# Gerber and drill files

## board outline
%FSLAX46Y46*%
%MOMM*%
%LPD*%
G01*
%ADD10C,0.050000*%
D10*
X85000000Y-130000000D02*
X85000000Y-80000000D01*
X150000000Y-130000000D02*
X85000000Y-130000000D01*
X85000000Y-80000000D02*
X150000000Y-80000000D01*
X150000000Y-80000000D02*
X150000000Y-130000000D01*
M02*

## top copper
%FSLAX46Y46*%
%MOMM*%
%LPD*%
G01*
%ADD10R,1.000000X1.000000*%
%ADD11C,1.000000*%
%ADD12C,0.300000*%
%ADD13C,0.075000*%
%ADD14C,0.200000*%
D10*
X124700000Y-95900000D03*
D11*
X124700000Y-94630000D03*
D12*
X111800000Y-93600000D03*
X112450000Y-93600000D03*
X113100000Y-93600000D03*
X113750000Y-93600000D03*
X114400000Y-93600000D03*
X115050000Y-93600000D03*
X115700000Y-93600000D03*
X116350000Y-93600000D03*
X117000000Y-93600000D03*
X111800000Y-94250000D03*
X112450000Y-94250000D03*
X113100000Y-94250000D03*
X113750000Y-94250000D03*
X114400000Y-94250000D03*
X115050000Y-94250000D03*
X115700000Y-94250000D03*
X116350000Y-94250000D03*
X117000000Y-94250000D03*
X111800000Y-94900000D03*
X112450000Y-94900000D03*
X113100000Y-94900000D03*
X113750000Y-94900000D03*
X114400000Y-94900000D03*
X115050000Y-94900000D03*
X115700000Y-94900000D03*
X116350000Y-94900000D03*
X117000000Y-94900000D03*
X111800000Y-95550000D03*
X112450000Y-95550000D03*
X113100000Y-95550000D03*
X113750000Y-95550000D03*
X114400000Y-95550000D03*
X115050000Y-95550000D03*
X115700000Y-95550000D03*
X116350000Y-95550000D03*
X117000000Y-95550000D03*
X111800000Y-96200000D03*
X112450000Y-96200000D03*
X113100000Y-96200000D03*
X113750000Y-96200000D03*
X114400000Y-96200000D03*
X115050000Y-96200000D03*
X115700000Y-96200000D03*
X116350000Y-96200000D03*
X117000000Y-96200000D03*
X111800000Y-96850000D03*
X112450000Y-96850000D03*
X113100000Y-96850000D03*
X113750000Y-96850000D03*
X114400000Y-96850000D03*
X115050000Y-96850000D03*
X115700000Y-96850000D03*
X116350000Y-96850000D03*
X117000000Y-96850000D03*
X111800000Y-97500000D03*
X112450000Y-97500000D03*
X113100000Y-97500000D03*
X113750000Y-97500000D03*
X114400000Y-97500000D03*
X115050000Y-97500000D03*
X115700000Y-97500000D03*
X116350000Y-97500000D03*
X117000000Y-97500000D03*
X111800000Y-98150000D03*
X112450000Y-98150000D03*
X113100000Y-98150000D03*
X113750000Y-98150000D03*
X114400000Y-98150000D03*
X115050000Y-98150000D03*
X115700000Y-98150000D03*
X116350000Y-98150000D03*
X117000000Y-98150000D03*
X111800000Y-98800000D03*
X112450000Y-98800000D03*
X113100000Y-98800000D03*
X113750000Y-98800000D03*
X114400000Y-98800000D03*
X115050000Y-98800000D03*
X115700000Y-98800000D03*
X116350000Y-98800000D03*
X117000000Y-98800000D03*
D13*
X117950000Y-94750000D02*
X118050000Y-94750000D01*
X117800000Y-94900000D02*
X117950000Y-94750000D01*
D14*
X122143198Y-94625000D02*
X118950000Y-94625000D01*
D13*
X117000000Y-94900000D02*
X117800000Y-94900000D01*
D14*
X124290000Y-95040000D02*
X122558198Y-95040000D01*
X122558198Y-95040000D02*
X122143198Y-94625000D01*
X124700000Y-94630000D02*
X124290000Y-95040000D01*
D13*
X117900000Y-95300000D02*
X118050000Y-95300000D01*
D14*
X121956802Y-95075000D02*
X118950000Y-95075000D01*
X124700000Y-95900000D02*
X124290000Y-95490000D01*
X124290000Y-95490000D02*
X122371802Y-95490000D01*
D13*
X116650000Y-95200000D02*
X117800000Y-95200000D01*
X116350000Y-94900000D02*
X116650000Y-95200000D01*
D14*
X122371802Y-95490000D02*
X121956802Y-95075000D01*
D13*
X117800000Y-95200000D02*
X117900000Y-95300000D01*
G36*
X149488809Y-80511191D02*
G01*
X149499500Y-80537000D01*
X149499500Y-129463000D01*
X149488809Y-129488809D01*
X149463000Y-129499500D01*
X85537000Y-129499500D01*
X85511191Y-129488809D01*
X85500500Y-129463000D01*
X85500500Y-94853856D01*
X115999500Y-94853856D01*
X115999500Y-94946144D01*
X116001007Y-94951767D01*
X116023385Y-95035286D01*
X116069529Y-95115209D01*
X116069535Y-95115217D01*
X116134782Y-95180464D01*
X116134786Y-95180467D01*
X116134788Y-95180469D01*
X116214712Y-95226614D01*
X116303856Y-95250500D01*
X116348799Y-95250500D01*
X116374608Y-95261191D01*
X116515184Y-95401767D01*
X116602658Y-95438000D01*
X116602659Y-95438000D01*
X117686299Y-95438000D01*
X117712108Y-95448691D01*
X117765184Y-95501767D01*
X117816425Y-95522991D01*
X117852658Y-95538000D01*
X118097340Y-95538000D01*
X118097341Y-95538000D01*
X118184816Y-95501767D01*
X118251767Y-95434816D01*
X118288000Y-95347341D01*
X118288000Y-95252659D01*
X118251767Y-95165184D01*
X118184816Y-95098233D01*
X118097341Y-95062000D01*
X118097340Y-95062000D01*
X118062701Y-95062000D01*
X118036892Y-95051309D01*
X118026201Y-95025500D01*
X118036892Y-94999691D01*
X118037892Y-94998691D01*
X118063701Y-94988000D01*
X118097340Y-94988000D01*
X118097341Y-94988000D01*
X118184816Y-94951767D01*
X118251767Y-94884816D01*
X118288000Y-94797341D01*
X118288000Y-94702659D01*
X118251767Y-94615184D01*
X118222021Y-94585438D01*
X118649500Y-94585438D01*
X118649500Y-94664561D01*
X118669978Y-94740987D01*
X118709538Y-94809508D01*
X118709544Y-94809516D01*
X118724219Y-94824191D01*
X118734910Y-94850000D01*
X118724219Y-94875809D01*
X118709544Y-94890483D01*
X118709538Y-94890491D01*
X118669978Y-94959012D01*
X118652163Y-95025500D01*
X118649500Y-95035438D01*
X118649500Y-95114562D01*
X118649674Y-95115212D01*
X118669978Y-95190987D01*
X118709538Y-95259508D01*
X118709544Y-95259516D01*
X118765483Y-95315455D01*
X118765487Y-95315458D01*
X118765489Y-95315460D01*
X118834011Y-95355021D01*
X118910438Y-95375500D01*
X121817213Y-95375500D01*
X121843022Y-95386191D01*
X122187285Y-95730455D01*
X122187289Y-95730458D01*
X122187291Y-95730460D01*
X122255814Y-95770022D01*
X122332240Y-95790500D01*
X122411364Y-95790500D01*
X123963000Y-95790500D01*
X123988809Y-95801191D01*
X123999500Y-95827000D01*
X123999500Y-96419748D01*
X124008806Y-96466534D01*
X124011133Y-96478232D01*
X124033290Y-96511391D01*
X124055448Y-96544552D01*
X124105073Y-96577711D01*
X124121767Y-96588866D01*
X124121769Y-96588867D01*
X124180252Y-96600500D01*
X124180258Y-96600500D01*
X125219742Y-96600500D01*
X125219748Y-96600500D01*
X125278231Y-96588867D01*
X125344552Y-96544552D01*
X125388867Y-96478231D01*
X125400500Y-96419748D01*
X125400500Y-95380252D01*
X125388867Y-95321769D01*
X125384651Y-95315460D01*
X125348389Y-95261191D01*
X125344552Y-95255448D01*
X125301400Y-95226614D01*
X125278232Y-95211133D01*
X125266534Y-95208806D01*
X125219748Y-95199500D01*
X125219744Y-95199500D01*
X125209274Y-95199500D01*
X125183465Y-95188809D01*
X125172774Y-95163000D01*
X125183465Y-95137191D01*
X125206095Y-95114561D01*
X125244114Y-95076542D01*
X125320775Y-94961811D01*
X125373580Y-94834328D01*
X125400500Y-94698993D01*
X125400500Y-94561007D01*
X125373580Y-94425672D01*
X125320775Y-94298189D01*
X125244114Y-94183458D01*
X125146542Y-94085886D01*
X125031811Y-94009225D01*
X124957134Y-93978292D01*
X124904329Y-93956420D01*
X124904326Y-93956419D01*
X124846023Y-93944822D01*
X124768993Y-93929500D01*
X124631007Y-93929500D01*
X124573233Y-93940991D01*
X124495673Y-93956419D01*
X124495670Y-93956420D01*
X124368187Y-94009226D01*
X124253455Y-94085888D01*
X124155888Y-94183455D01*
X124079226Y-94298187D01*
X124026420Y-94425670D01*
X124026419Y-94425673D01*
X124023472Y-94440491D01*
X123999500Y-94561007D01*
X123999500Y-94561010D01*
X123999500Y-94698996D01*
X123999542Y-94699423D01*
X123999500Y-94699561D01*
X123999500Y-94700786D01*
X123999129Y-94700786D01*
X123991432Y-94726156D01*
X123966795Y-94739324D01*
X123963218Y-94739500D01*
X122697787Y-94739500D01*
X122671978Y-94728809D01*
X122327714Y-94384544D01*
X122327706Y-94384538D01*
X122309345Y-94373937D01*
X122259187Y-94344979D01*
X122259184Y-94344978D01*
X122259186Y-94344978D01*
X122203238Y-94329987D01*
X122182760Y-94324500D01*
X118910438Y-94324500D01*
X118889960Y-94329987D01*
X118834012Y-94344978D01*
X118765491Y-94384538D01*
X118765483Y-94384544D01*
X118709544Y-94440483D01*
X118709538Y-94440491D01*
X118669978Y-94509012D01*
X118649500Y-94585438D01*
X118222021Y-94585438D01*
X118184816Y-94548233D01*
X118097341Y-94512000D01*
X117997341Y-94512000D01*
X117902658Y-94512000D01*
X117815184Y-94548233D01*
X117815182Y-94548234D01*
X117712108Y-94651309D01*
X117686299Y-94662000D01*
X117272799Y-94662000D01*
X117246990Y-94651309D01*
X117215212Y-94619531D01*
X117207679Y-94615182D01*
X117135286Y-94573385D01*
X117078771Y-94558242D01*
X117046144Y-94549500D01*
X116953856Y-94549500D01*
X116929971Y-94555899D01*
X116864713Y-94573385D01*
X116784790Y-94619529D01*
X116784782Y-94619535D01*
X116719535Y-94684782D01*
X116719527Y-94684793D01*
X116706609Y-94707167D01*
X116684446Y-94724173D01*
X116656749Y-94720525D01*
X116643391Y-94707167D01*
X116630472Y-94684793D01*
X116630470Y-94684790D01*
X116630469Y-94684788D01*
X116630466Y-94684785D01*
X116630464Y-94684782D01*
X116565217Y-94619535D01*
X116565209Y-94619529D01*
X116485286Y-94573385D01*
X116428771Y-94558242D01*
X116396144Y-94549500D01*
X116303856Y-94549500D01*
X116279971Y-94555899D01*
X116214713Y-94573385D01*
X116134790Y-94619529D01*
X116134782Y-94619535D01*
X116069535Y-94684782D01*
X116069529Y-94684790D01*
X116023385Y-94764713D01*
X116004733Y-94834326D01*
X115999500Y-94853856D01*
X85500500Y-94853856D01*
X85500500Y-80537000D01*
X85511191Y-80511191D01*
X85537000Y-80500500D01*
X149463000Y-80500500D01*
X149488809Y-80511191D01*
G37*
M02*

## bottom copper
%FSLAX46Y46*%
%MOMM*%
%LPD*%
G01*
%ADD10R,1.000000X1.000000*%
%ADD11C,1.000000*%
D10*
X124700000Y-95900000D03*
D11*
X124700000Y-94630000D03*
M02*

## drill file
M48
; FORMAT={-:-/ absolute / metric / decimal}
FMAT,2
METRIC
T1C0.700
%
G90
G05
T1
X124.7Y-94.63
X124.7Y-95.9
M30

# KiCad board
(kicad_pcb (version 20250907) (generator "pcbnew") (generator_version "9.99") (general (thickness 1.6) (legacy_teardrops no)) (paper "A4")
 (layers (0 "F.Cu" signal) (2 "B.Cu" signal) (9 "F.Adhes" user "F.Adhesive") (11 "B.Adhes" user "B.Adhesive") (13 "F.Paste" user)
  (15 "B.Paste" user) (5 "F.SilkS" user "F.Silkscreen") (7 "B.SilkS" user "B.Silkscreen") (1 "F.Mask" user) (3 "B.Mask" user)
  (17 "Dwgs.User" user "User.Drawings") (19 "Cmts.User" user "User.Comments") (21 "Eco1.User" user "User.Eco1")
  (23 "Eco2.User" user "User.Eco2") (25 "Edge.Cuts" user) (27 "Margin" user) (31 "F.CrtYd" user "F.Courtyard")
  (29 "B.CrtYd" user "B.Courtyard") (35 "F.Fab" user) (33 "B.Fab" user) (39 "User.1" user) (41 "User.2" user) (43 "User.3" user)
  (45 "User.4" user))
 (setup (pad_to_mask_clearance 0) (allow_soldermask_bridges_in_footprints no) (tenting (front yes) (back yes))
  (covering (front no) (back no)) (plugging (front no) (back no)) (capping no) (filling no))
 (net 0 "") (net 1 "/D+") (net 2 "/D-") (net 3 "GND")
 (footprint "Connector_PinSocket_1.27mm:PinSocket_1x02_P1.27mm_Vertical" (layer "F.Cu") (at 124.7 95.9 180)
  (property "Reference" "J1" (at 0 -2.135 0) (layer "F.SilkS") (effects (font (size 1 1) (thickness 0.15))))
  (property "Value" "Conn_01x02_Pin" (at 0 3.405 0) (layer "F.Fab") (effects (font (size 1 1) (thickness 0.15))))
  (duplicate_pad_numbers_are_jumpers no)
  (pad "1" thru_hole rect (at 0 0 180) (size 1 1) (drill 0.7) (layers "*.Cu" "*.Mask") (remove_unused_layers no) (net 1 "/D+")
   (tenting (front none) (back none)))
  (pad "2" thru_hole circle (at 0 1.27 180) (size 1 1) (drill 0.7) (layers "*.Cu" "*.Mask") (remove_unused_layers no) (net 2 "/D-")
   (tenting (front none) (back none))))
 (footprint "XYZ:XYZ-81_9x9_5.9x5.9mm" (layer "F.Cu") (at 114.4 96.2)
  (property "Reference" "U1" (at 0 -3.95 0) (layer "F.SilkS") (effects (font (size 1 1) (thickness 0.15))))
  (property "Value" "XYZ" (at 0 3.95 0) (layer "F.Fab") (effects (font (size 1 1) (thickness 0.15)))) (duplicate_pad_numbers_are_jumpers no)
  (pad "A1" smd circle (at -2.6 -2.6) (size 0.3 0.3) (layers "F.Cu" "F.Mask" "F.Paste") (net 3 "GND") (tenting (front none) (back none)))
  (pad "A2" smd circle (at -1.95 -2.6) (size 0.3 0.3) (layers "F.Cu" "F.Mask" "F.Paste") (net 3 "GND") (tenting (front none) (back none)))
  (pad "A3" smd circle (at -1.3 -2.6) (size 0.3 0.3) (layers "F.Cu" "F.Mask" "F.Paste") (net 3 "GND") (tenting (front none) (back none)))
  (pad "A4" smd circle (at -0.65 -2.6) (size 0.3 0.3) (layers "F.Cu" "F.Mask" "F.Paste") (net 3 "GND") (tenting (front none) (back none)))
  (pad "A5" smd circle (at 0 -2.6) (size 0.3 0.3) (layers "F.Cu" "F.Mask" "F.Paste") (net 3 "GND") (tenting (front none) (back none)))
  (pad "A6" smd circle (at 0.65 -2.6) (size 0.3 0.3) (layers "F.Cu" "F.Mask" "F.Paste") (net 3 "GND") (tenting (front none) (back none)))
  (pad "A7" smd circle (at 1.3 -2.6) (size 0.3 0.3) (layers "F.Cu" "F.Mask" "F.Paste") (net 3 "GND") (tenting (front none) (back none)))
  (pad "A8" smd circle (at 1.95 -2.6) (size 0.3 0.3) (layers "F.Cu" "F.Mask" "F.Paste") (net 3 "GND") (tenting (front none) (back none)))
  (pad "A9" smd circle (at 2.6 -2.6) (size 0.3 0.3) (layers "F.Cu" "F.Mask" "F.Paste") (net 3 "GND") (tenting (front none) (back none)))
  (pad "B1" smd circle (at -2.6 -1.95) (size 0.3 0.3) (layers "F.Cu" "F.Mask" "F.Paste") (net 3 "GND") (tenting (front none) (back none)))
  (pad "B2" smd circle (at -1.95 -1.95) (size 0.3 0.3) (layers "F.Cu" "F.Mask" "F.Paste") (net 3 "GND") (tenting (front none) (back none)))
  (pad "B3" smd circle (at -1.3 -1.95) (size 0.3 0.3) (layers "F.Cu" "F.Mask" "F.Paste") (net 3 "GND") (tenting (front none) (back none)))
  (pad "B4" smd circle (at -0.65 -1.95) (size 0.3 0.3) (layers "F.Cu" "F.Mask" "F.Paste") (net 3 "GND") (tenting (front none) (back none)))
  (pad "B5" smd circle (at 0 -1.95) (size 0.3 0.3) (layers "F.Cu" "F.Mask" "F.Paste") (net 3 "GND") (tenting (front none) (back none)))
  (pad "B6" smd circle (at 0.65 -1.95) (size 0.3 0.3) (layers "F.Cu" "F.Mask" "F.Paste") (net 3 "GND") (tenting (front none) (back none)))
  (pad "B7" smd circle (at 1.3 -1.95) (size 0.3 0.3) (layers "F.Cu" "F.Mask" "F.Paste") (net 3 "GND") (tenting (front none) (back none)))
  (pad "B8" smd circle (at 1.95 -1.95) (size 0.3 0.3) (layers "F.Cu" "F.Mask" "F.Paste") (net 3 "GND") (tenting (front none) (back none)))
  (pad "B9" smd circle (at 2.6 -1.95) (size 0.3 0.3) (layers "F.Cu" "F.Mask" "F.Paste") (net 3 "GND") (tenting (front none) (back none)))
  (pad "C1" smd circle (at -2.6 -1.3) (size 0.3 0.3) (layers "F.Cu" "F.Mask" "F.Paste") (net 3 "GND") (tenting (front none) (back none)))
  (pad "C2" smd circle (at -1.95 -1.3) (size 0.3 0.3) (layers "F.Cu" "F.Mask" "F.Paste") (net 3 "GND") (tenting (front none) (back none)))
  (pad "C3" smd circle (at -1.3 -1.3) (size 0.3 0.3) (layers "F.Cu" "F.Mask" "F.Paste") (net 3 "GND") (tenting (front none) (back none)))
  (pad "C4" smd circle (at -0.65 -1.3) (size 0.3 0.3) (layers "F.Cu" "F.Mask" "F.Paste") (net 3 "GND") (tenting (front none) (back none)))
  (pad "C5" smd circle (at 0 -1.3) (size 0.3 0.3) (layers "F.Cu" "F.Mask" "F.Paste") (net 3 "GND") (tenting (front none) (back none)))
  (pad "C6" smd circle (at 0.65 -1.3) (size 0.3 0.3) (layers "F.Cu" "F.Mask" "F.Paste") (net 3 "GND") (tenting (front none) (back none)))
  (pad "C7" smd circle (at 1.3 -1.3) (size 0.3 0.3) (layers "F.Cu" "F.Mask" "F.Paste") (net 3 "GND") (tenting (front none) (back none)))
  (pad "C8" smd circle (at 1.95 -1.3) (size 0.3 0.3) (layers "F.Cu" "F.Mask" "F.Paste") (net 1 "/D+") (tenting (front none) (back none)))
  (pad "C9" smd circle (at 2.6 -1.3) (size 0.3 0.3) (layers "F.Cu" "F.Mask" "F.Paste") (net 2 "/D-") (tenting (front none) (back none)))
  (pad "D1" smd circle (at -2.6 -0.65) (size 0.3 0.3) (layers "F.Cu" "F.Mask" "F.Paste") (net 3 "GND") (tenting (front none) (back none)))
  (pad "D2" smd circle (at -1.95 -0.65) (size 0.3 0.3) (layers "F.Cu" "F.Mask" "F.Paste") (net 3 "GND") (tenting (front none) (back none)))
  (pad "D3" smd circle (at -1.3 -0.65) (size 0.3 0.3) (layers "F.Cu" "F.Mask" "F.Paste") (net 3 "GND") (tenting (front none) (back none)))
  (pad "D4" smd circle (at -0.65 -0.65) (size 0.3 0.3) (layers "F.Cu" "F.Mask" "F.Paste") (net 3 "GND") (tenting (front none) (back none)))
  (pad "D5" smd circle (at 0 -0.65) (size 0.3 0.3) (layers "F.Cu" "F.Mask" "F.Paste") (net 3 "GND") (tenting (front none) (back none)))
  (pad "D6" smd circle (at 0.65 -0.65) (size 0.3 0.3) (layers "F.Cu" "F.Mask" "F.Paste") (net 3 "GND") (tenting (front none) (back none)))
  (pad "D7" smd circle (at 1.3 -0.65) (size 0.3 0.3) (layers "F.Cu" "F.Mask" "F.Paste") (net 3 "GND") (tenting (front none) (back none)))
  (pad "D8" smd circle (at 1.95 -0.65) (size 0.3 0.3) (layers "F.Cu" "F.Mask" "F.Paste") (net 3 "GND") (tenting (front none) (back none)))
  (pad "D9" smd circle (at 2.6 -0.65) (size 0.3 0.3) (layers "F.Cu" "F.Mask" "F.Paste") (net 3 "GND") (tenting (front none) (back none)))
  (pad "E1" smd circle (at -2.6 0) (size 0.3 0.3) (layers "F.Cu" "F.Mask" "F.Paste") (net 3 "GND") (tenting (front none) (back none)))
  (pad "E2" smd circle (at -1.95 0) (size 0.3 0.3) (layers "F.Cu" "F.Mask" "F.Paste") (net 3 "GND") (tenting (front none) (back none)))
  (pad "E3" smd circle (at -1.3 0) (size 0.3 0.3) (layers "F.Cu" "F.Mask" "F.Paste") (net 3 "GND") (tenting (front none) (back none)))
  (pad "E4" smd circle (at -0.65 0) (size 0.3 0.3) (layers "F.Cu" "F.Mask" "F.Paste") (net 3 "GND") (tenting (front none) (back none)))
  (pad "E5" smd circle (at 0 0) (size 0.3 0.3) (layers "F.Cu" "F.Mask" "F.Paste") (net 3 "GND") (tenting (front none) (back none)))
  (pad "E6" smd circle (at 0.65 0) (size 0.3 0.3) (layers "F.Cu" "F.Mask" "F.Paste") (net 3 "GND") (tenting (front none) (back none)))
  (pad "E7" smd circle (at 1.3 0) (size 0.3 0.3) (layers "F.Cu" "F.Mask" "F.Paste") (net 3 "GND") (tenting (front none) (back none)))
  (pad "E8" smd circle (at 1.95 0) (size 0.3 0.3) (layers "F.Cu" "F.Mask" "F.Paste") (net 3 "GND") (tenting (front none) (back none)))
  (pad "E9" smd circle (at 2.6 0) (size 0.3 0.3) (layers "F.Cu" "F.Mask" "F.Paste") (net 3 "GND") (tenting (front none) (back none)))
  (pad "F1" smd circle (at -2.6 0.65) (size 0.3 0.3) (layers "F.Cu" "F.Mask" "F.Paste") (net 3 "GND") (tenting (front none) (back none)))
  (pad "F2" smd circle (at -1.95 0.65) (size 0.3 0.3) (layers "F.Cu" "F.Mask" "F.Paste") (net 3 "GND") (tenting (front none) (back none)))
  (pad "F3" smd circle (at -1.3 0.65) (size 0.3 0.3) (layers "F.Cu" "F.Mask" "F.Paste") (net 3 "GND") (tenting (front none) (back none)))
  (pad "F4" smd circle (at -0.65 0.65) (size 0.3 0.3) (layers "F.Cu" "F.Mask" "F.Paste") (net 3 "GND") (tenting (front none) (back none)))
  (pad "F5" smd circle (at 0 0.65) (size 0.3 0.3) (layers "F.Cu" "F.Mask" "F.Paste") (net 3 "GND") (tenting (front none) (back none)))
  (pad "F6" smd circle (at 0.65 0.65) (size 0.3 0.3) (layers "F.Cu" "F.Mask" "F.Paste") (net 3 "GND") (tenting (front none) (back none)))
  (pad "F7" smd circle (at 1.3 0.65) (size 0.3 0.3) (layers "F.Cu" "F.Mask" "F.Paste") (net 3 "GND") (tenting (front none) (back none)))
  (pad "F8" smd circle (at 1.95 0.65) (size 0.3 0.3) (layers "F.Cu" "F.Mask" "F.Paste") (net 3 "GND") (tenting (front none) (back none)))
  (pad "F9" smd circle (at 2.6 0.65) (size 0.3 0.3) (layers "F.Cu" "F.Mask" "F.Paste") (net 3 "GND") (tenting (front none) (back none)))
  (pad "G1" smd circle (at -2.6 1.3) (size 0.3 0.3) (layers "F.Cu" "F.Mask" "F.Paste") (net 3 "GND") (tenting (front none) (back none)))
  (pad "G2" smd circle (at -1.95 1.3) (size 0.3 0.3) (layers "F.Cu" "F.Mask" "F.Paste") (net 3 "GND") (tenting (front none) (back none)))
  (pad "G3" smd circle (at -1.3 1.3) (size 0.3 0.3) (layers "F.Cu" "F.Mask" "F.Paste") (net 3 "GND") (tenting (front none) (back none)))
  (pad "G4" smd circle (at -0.65 1.3) (size 0.3 0.3) (layers "F.Cu" "F.Mask" "F.Paste") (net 3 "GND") (tenting (front none) (back none)))
  (pad "G5" smd circle (at 0 1.3) (size 0.3 0.3) (layers "F.Cu" "F.Mask" "F.Paste") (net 3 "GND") (tenting (front none) (back none)))
  (pad "G6" smd circle (at 0.65 1.3) (size 0.3 0.3) (layers "F.Cu" "F.Mask" "F.Paste") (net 3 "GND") (tenting (front none) (back none)))
  (pad "G7" smd circle (at 1.3 1.3) (size 0.3 0.3) (layers "F.Cu" "F.Mask" "F.Paste") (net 3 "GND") (tenting (front none) (back none)))
  (pad "G8" smd circle (at 1.95 1.3) (size 0.3 0.3) (layers "F.Cu" "F.Mask" "F.Paste") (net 3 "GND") (tenting (front none) (back none)))
  (pad "G9" smd circle (at 2.6 1.3) (size 0.3 0.3) (layers "F.Cu" "F.Mask" "F.Paste") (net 3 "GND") (tenting (front none) (back none)))
  (pad "H1" smd circle (at -2.6 1.95) (size 0.3 0.3) (layers "F.Cu" "F.Mask" "F.Paste") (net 3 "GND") (tenting (front none) (back none)))
  (pad "H2" smd circle (at -1.95 1.95) (size 0.3 0.3) (layers "F.Cu" "F.Mask" "F.Paste") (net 3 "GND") (tenting (front none) (back none)))
  (pad "H3" smd circle (at -1.3 1.95) (size 0.3 0.3) (layers "F.Cu" "F.Mask" "F.Paste") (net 3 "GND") (tenting (front none) (back none)))
  (pad "H4" smd circle (at -0.65 1.95) (size 0.3 0.3) (layers "F.Cu" "F.Mask" "F.Paste") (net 3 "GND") (tenting (front none) (back none)))
  (pad "H5" smd circle (at 0 1.95) (size 0.3 0.3) (layers "F.Cu" "F.Mask" "F.Paste") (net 3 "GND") (tenting (front none) (back none)))
  (pad "H6" smd circle (at 0.65 1.95) (size 0.3 0.3) (layers "F.Cu" "F.Mask" "F.Paste") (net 3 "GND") (tenting (front none) (back none)))
  (pad "H7" smd circle (at 1.3 1.95) (size 0.3 0.3) (layers "F.Cu" "F.Mask" "F.Paste") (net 3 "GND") (tenting (front none) (back none)))
  (pad "H8" smd circle (at 1.95 1.95) (size 0.3 0.3) (layers "F.Cu" "F.Mask" "F.Paste") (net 3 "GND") (tenting (front none) (back none)))
  (pad "H9" smd circle (at 2.6 1.95) (size 0.3 0.3) (layers "F.Cu" "F.Mask" "F.Paste") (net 3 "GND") (tenting (front none) (back none)))
  (pad "J1" smd circle (at -2.6 2.6) (size 0.3 0.3) (layers "F.Cu" "F.Mask" "F.Paste") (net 3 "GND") (tenting (front none) (back none)))
  (pad "J2" smd circle (at -1.95 2.6) (size 0.3 0.3) (layers "F.Cu" "F.Mask" "F.Paste") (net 3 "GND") (tenting (front none) (back none)))
  (pad "J3" smd circle (at -1.3 2.6) (size 0.3 0.3) (layers "F.Cu" "F.Mask" "F.Paste") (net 3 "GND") (tenting (front none) (back none)))
  (pad "J4" smd circle (at -0.65 2.6) (size 0.3 0.3) (layers "F.Cu" "F.Mask" "F.Paste") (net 3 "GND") (tenting (front none) (back none)))
  (pad "J5" smd circle (at 0 2.6) (size 0.3 0.3) (layers "F.Cu" "F.Mask" "F.Paste") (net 3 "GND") (tenting (front none) (back none)))
  (pad "J6" smd circle (at 0.65 2.6) (size 0.3 0.3) (layers "F.Cu" "F.Mask" "F.Paste") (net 3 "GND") (tenting (front none) (back none)))
  (pad "J7" smd circle (at 1.3 2.6) (size 0.3 0.3) (layers "F.Cu" "F.Mask" "F.Paste") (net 3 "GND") (tenting (front none) (back none)))
  (pad "J8" smd circle (at 1.95 2.6) (size 0.3 0.3) (layers "F.Cu" "F.Mask" "F.Paste") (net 3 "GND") (tenting (front none) (back none)))
  (pad "J9" smd circle (at 2.6 2.6) (size 0.3 0.3) (layers "F.Cu" "F.Mask" "F.Paste") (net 3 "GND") (tenting (front none) (back none))))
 (gr_line (start 85 130) (end 85 80) (stroke (width 0.05) (type default)) (layer "Edge.Cuts"))
 (gr_line (start 150 130) (end 85 130) (stroke (width 0.05) (type default)) (layer "Edge.Cuts"))
 (gr_line (start 85 80) (end 150 80) (stroke (width 0.05) (type default)) (layer "Edge.Cuts"))
 (gr_line (start 150 80) (end 150 130) (stroke (width 0.05) (type default)) (layer "Edge.Cuts"))
 (segment (start 117.95 94.75) (end 118.05 94.75) (width 0.075) (layer "F.Cu") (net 2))
 (segment (start 117.8 94.9) (end 117.95 94.75) (width 0.075) (layer "F.Cu") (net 2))
 (segment (start 122.143198 94.625) (end 118.95 94.625) (width 0.2) (layer "F.Cu") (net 2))
 (segment (start 117 94.9) (end 117.8 94.9) (width 0.075) (layer "F.Cu") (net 2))
 (segment (start 124.29 95.04) (end 122.558198 95.04) (width 0.2) (layer "F.Cu") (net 2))
 (segment (start 122.558198 95.04) (end 122.143198 94.625) (width 0.2) (layer "F.Cu") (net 2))
 (segment (start 124.7 94.63) (end 124.29 95.04) (width 0.2) (layer "F.Cu") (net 2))
 (segment (start 117.9 95.3) (end 118.05 95.3) (width 0.075) (layer "F.Cu") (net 1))
 (segment (start 121.956802 95.075) (end 118.95 95.075) (width 0.2) (layer "F.Cu") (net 1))
 (segment (start 124.7 95.9) (end 124.29 95.49) (width 0.2) (layer "F.Cu") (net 1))
 (segment (start 124.29 95.49) (end 122.371802 95.49) (width 0.2) (layer "F.Cu") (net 1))
 (segment (start 116.65 95.2) (end 117.8 95.2) (width 0.075) (layer "F.Cu") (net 1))
 (segment (start 116.35 94.9) (end 116.65 95.2) (width 0.075) (layer "F.Cu") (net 1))
 (segment (start 122.371802 95.49) (end 121.956802 95.075) (width 0.2) (layer "F.Cu") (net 1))
 (segment (start 117.8 95.2) (end 117.9 95.3) (width 0.075) (layer "F.Cu") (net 1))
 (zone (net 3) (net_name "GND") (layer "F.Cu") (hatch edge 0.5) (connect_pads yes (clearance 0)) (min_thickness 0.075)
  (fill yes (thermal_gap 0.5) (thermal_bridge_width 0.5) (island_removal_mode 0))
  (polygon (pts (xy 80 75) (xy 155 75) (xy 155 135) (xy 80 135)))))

